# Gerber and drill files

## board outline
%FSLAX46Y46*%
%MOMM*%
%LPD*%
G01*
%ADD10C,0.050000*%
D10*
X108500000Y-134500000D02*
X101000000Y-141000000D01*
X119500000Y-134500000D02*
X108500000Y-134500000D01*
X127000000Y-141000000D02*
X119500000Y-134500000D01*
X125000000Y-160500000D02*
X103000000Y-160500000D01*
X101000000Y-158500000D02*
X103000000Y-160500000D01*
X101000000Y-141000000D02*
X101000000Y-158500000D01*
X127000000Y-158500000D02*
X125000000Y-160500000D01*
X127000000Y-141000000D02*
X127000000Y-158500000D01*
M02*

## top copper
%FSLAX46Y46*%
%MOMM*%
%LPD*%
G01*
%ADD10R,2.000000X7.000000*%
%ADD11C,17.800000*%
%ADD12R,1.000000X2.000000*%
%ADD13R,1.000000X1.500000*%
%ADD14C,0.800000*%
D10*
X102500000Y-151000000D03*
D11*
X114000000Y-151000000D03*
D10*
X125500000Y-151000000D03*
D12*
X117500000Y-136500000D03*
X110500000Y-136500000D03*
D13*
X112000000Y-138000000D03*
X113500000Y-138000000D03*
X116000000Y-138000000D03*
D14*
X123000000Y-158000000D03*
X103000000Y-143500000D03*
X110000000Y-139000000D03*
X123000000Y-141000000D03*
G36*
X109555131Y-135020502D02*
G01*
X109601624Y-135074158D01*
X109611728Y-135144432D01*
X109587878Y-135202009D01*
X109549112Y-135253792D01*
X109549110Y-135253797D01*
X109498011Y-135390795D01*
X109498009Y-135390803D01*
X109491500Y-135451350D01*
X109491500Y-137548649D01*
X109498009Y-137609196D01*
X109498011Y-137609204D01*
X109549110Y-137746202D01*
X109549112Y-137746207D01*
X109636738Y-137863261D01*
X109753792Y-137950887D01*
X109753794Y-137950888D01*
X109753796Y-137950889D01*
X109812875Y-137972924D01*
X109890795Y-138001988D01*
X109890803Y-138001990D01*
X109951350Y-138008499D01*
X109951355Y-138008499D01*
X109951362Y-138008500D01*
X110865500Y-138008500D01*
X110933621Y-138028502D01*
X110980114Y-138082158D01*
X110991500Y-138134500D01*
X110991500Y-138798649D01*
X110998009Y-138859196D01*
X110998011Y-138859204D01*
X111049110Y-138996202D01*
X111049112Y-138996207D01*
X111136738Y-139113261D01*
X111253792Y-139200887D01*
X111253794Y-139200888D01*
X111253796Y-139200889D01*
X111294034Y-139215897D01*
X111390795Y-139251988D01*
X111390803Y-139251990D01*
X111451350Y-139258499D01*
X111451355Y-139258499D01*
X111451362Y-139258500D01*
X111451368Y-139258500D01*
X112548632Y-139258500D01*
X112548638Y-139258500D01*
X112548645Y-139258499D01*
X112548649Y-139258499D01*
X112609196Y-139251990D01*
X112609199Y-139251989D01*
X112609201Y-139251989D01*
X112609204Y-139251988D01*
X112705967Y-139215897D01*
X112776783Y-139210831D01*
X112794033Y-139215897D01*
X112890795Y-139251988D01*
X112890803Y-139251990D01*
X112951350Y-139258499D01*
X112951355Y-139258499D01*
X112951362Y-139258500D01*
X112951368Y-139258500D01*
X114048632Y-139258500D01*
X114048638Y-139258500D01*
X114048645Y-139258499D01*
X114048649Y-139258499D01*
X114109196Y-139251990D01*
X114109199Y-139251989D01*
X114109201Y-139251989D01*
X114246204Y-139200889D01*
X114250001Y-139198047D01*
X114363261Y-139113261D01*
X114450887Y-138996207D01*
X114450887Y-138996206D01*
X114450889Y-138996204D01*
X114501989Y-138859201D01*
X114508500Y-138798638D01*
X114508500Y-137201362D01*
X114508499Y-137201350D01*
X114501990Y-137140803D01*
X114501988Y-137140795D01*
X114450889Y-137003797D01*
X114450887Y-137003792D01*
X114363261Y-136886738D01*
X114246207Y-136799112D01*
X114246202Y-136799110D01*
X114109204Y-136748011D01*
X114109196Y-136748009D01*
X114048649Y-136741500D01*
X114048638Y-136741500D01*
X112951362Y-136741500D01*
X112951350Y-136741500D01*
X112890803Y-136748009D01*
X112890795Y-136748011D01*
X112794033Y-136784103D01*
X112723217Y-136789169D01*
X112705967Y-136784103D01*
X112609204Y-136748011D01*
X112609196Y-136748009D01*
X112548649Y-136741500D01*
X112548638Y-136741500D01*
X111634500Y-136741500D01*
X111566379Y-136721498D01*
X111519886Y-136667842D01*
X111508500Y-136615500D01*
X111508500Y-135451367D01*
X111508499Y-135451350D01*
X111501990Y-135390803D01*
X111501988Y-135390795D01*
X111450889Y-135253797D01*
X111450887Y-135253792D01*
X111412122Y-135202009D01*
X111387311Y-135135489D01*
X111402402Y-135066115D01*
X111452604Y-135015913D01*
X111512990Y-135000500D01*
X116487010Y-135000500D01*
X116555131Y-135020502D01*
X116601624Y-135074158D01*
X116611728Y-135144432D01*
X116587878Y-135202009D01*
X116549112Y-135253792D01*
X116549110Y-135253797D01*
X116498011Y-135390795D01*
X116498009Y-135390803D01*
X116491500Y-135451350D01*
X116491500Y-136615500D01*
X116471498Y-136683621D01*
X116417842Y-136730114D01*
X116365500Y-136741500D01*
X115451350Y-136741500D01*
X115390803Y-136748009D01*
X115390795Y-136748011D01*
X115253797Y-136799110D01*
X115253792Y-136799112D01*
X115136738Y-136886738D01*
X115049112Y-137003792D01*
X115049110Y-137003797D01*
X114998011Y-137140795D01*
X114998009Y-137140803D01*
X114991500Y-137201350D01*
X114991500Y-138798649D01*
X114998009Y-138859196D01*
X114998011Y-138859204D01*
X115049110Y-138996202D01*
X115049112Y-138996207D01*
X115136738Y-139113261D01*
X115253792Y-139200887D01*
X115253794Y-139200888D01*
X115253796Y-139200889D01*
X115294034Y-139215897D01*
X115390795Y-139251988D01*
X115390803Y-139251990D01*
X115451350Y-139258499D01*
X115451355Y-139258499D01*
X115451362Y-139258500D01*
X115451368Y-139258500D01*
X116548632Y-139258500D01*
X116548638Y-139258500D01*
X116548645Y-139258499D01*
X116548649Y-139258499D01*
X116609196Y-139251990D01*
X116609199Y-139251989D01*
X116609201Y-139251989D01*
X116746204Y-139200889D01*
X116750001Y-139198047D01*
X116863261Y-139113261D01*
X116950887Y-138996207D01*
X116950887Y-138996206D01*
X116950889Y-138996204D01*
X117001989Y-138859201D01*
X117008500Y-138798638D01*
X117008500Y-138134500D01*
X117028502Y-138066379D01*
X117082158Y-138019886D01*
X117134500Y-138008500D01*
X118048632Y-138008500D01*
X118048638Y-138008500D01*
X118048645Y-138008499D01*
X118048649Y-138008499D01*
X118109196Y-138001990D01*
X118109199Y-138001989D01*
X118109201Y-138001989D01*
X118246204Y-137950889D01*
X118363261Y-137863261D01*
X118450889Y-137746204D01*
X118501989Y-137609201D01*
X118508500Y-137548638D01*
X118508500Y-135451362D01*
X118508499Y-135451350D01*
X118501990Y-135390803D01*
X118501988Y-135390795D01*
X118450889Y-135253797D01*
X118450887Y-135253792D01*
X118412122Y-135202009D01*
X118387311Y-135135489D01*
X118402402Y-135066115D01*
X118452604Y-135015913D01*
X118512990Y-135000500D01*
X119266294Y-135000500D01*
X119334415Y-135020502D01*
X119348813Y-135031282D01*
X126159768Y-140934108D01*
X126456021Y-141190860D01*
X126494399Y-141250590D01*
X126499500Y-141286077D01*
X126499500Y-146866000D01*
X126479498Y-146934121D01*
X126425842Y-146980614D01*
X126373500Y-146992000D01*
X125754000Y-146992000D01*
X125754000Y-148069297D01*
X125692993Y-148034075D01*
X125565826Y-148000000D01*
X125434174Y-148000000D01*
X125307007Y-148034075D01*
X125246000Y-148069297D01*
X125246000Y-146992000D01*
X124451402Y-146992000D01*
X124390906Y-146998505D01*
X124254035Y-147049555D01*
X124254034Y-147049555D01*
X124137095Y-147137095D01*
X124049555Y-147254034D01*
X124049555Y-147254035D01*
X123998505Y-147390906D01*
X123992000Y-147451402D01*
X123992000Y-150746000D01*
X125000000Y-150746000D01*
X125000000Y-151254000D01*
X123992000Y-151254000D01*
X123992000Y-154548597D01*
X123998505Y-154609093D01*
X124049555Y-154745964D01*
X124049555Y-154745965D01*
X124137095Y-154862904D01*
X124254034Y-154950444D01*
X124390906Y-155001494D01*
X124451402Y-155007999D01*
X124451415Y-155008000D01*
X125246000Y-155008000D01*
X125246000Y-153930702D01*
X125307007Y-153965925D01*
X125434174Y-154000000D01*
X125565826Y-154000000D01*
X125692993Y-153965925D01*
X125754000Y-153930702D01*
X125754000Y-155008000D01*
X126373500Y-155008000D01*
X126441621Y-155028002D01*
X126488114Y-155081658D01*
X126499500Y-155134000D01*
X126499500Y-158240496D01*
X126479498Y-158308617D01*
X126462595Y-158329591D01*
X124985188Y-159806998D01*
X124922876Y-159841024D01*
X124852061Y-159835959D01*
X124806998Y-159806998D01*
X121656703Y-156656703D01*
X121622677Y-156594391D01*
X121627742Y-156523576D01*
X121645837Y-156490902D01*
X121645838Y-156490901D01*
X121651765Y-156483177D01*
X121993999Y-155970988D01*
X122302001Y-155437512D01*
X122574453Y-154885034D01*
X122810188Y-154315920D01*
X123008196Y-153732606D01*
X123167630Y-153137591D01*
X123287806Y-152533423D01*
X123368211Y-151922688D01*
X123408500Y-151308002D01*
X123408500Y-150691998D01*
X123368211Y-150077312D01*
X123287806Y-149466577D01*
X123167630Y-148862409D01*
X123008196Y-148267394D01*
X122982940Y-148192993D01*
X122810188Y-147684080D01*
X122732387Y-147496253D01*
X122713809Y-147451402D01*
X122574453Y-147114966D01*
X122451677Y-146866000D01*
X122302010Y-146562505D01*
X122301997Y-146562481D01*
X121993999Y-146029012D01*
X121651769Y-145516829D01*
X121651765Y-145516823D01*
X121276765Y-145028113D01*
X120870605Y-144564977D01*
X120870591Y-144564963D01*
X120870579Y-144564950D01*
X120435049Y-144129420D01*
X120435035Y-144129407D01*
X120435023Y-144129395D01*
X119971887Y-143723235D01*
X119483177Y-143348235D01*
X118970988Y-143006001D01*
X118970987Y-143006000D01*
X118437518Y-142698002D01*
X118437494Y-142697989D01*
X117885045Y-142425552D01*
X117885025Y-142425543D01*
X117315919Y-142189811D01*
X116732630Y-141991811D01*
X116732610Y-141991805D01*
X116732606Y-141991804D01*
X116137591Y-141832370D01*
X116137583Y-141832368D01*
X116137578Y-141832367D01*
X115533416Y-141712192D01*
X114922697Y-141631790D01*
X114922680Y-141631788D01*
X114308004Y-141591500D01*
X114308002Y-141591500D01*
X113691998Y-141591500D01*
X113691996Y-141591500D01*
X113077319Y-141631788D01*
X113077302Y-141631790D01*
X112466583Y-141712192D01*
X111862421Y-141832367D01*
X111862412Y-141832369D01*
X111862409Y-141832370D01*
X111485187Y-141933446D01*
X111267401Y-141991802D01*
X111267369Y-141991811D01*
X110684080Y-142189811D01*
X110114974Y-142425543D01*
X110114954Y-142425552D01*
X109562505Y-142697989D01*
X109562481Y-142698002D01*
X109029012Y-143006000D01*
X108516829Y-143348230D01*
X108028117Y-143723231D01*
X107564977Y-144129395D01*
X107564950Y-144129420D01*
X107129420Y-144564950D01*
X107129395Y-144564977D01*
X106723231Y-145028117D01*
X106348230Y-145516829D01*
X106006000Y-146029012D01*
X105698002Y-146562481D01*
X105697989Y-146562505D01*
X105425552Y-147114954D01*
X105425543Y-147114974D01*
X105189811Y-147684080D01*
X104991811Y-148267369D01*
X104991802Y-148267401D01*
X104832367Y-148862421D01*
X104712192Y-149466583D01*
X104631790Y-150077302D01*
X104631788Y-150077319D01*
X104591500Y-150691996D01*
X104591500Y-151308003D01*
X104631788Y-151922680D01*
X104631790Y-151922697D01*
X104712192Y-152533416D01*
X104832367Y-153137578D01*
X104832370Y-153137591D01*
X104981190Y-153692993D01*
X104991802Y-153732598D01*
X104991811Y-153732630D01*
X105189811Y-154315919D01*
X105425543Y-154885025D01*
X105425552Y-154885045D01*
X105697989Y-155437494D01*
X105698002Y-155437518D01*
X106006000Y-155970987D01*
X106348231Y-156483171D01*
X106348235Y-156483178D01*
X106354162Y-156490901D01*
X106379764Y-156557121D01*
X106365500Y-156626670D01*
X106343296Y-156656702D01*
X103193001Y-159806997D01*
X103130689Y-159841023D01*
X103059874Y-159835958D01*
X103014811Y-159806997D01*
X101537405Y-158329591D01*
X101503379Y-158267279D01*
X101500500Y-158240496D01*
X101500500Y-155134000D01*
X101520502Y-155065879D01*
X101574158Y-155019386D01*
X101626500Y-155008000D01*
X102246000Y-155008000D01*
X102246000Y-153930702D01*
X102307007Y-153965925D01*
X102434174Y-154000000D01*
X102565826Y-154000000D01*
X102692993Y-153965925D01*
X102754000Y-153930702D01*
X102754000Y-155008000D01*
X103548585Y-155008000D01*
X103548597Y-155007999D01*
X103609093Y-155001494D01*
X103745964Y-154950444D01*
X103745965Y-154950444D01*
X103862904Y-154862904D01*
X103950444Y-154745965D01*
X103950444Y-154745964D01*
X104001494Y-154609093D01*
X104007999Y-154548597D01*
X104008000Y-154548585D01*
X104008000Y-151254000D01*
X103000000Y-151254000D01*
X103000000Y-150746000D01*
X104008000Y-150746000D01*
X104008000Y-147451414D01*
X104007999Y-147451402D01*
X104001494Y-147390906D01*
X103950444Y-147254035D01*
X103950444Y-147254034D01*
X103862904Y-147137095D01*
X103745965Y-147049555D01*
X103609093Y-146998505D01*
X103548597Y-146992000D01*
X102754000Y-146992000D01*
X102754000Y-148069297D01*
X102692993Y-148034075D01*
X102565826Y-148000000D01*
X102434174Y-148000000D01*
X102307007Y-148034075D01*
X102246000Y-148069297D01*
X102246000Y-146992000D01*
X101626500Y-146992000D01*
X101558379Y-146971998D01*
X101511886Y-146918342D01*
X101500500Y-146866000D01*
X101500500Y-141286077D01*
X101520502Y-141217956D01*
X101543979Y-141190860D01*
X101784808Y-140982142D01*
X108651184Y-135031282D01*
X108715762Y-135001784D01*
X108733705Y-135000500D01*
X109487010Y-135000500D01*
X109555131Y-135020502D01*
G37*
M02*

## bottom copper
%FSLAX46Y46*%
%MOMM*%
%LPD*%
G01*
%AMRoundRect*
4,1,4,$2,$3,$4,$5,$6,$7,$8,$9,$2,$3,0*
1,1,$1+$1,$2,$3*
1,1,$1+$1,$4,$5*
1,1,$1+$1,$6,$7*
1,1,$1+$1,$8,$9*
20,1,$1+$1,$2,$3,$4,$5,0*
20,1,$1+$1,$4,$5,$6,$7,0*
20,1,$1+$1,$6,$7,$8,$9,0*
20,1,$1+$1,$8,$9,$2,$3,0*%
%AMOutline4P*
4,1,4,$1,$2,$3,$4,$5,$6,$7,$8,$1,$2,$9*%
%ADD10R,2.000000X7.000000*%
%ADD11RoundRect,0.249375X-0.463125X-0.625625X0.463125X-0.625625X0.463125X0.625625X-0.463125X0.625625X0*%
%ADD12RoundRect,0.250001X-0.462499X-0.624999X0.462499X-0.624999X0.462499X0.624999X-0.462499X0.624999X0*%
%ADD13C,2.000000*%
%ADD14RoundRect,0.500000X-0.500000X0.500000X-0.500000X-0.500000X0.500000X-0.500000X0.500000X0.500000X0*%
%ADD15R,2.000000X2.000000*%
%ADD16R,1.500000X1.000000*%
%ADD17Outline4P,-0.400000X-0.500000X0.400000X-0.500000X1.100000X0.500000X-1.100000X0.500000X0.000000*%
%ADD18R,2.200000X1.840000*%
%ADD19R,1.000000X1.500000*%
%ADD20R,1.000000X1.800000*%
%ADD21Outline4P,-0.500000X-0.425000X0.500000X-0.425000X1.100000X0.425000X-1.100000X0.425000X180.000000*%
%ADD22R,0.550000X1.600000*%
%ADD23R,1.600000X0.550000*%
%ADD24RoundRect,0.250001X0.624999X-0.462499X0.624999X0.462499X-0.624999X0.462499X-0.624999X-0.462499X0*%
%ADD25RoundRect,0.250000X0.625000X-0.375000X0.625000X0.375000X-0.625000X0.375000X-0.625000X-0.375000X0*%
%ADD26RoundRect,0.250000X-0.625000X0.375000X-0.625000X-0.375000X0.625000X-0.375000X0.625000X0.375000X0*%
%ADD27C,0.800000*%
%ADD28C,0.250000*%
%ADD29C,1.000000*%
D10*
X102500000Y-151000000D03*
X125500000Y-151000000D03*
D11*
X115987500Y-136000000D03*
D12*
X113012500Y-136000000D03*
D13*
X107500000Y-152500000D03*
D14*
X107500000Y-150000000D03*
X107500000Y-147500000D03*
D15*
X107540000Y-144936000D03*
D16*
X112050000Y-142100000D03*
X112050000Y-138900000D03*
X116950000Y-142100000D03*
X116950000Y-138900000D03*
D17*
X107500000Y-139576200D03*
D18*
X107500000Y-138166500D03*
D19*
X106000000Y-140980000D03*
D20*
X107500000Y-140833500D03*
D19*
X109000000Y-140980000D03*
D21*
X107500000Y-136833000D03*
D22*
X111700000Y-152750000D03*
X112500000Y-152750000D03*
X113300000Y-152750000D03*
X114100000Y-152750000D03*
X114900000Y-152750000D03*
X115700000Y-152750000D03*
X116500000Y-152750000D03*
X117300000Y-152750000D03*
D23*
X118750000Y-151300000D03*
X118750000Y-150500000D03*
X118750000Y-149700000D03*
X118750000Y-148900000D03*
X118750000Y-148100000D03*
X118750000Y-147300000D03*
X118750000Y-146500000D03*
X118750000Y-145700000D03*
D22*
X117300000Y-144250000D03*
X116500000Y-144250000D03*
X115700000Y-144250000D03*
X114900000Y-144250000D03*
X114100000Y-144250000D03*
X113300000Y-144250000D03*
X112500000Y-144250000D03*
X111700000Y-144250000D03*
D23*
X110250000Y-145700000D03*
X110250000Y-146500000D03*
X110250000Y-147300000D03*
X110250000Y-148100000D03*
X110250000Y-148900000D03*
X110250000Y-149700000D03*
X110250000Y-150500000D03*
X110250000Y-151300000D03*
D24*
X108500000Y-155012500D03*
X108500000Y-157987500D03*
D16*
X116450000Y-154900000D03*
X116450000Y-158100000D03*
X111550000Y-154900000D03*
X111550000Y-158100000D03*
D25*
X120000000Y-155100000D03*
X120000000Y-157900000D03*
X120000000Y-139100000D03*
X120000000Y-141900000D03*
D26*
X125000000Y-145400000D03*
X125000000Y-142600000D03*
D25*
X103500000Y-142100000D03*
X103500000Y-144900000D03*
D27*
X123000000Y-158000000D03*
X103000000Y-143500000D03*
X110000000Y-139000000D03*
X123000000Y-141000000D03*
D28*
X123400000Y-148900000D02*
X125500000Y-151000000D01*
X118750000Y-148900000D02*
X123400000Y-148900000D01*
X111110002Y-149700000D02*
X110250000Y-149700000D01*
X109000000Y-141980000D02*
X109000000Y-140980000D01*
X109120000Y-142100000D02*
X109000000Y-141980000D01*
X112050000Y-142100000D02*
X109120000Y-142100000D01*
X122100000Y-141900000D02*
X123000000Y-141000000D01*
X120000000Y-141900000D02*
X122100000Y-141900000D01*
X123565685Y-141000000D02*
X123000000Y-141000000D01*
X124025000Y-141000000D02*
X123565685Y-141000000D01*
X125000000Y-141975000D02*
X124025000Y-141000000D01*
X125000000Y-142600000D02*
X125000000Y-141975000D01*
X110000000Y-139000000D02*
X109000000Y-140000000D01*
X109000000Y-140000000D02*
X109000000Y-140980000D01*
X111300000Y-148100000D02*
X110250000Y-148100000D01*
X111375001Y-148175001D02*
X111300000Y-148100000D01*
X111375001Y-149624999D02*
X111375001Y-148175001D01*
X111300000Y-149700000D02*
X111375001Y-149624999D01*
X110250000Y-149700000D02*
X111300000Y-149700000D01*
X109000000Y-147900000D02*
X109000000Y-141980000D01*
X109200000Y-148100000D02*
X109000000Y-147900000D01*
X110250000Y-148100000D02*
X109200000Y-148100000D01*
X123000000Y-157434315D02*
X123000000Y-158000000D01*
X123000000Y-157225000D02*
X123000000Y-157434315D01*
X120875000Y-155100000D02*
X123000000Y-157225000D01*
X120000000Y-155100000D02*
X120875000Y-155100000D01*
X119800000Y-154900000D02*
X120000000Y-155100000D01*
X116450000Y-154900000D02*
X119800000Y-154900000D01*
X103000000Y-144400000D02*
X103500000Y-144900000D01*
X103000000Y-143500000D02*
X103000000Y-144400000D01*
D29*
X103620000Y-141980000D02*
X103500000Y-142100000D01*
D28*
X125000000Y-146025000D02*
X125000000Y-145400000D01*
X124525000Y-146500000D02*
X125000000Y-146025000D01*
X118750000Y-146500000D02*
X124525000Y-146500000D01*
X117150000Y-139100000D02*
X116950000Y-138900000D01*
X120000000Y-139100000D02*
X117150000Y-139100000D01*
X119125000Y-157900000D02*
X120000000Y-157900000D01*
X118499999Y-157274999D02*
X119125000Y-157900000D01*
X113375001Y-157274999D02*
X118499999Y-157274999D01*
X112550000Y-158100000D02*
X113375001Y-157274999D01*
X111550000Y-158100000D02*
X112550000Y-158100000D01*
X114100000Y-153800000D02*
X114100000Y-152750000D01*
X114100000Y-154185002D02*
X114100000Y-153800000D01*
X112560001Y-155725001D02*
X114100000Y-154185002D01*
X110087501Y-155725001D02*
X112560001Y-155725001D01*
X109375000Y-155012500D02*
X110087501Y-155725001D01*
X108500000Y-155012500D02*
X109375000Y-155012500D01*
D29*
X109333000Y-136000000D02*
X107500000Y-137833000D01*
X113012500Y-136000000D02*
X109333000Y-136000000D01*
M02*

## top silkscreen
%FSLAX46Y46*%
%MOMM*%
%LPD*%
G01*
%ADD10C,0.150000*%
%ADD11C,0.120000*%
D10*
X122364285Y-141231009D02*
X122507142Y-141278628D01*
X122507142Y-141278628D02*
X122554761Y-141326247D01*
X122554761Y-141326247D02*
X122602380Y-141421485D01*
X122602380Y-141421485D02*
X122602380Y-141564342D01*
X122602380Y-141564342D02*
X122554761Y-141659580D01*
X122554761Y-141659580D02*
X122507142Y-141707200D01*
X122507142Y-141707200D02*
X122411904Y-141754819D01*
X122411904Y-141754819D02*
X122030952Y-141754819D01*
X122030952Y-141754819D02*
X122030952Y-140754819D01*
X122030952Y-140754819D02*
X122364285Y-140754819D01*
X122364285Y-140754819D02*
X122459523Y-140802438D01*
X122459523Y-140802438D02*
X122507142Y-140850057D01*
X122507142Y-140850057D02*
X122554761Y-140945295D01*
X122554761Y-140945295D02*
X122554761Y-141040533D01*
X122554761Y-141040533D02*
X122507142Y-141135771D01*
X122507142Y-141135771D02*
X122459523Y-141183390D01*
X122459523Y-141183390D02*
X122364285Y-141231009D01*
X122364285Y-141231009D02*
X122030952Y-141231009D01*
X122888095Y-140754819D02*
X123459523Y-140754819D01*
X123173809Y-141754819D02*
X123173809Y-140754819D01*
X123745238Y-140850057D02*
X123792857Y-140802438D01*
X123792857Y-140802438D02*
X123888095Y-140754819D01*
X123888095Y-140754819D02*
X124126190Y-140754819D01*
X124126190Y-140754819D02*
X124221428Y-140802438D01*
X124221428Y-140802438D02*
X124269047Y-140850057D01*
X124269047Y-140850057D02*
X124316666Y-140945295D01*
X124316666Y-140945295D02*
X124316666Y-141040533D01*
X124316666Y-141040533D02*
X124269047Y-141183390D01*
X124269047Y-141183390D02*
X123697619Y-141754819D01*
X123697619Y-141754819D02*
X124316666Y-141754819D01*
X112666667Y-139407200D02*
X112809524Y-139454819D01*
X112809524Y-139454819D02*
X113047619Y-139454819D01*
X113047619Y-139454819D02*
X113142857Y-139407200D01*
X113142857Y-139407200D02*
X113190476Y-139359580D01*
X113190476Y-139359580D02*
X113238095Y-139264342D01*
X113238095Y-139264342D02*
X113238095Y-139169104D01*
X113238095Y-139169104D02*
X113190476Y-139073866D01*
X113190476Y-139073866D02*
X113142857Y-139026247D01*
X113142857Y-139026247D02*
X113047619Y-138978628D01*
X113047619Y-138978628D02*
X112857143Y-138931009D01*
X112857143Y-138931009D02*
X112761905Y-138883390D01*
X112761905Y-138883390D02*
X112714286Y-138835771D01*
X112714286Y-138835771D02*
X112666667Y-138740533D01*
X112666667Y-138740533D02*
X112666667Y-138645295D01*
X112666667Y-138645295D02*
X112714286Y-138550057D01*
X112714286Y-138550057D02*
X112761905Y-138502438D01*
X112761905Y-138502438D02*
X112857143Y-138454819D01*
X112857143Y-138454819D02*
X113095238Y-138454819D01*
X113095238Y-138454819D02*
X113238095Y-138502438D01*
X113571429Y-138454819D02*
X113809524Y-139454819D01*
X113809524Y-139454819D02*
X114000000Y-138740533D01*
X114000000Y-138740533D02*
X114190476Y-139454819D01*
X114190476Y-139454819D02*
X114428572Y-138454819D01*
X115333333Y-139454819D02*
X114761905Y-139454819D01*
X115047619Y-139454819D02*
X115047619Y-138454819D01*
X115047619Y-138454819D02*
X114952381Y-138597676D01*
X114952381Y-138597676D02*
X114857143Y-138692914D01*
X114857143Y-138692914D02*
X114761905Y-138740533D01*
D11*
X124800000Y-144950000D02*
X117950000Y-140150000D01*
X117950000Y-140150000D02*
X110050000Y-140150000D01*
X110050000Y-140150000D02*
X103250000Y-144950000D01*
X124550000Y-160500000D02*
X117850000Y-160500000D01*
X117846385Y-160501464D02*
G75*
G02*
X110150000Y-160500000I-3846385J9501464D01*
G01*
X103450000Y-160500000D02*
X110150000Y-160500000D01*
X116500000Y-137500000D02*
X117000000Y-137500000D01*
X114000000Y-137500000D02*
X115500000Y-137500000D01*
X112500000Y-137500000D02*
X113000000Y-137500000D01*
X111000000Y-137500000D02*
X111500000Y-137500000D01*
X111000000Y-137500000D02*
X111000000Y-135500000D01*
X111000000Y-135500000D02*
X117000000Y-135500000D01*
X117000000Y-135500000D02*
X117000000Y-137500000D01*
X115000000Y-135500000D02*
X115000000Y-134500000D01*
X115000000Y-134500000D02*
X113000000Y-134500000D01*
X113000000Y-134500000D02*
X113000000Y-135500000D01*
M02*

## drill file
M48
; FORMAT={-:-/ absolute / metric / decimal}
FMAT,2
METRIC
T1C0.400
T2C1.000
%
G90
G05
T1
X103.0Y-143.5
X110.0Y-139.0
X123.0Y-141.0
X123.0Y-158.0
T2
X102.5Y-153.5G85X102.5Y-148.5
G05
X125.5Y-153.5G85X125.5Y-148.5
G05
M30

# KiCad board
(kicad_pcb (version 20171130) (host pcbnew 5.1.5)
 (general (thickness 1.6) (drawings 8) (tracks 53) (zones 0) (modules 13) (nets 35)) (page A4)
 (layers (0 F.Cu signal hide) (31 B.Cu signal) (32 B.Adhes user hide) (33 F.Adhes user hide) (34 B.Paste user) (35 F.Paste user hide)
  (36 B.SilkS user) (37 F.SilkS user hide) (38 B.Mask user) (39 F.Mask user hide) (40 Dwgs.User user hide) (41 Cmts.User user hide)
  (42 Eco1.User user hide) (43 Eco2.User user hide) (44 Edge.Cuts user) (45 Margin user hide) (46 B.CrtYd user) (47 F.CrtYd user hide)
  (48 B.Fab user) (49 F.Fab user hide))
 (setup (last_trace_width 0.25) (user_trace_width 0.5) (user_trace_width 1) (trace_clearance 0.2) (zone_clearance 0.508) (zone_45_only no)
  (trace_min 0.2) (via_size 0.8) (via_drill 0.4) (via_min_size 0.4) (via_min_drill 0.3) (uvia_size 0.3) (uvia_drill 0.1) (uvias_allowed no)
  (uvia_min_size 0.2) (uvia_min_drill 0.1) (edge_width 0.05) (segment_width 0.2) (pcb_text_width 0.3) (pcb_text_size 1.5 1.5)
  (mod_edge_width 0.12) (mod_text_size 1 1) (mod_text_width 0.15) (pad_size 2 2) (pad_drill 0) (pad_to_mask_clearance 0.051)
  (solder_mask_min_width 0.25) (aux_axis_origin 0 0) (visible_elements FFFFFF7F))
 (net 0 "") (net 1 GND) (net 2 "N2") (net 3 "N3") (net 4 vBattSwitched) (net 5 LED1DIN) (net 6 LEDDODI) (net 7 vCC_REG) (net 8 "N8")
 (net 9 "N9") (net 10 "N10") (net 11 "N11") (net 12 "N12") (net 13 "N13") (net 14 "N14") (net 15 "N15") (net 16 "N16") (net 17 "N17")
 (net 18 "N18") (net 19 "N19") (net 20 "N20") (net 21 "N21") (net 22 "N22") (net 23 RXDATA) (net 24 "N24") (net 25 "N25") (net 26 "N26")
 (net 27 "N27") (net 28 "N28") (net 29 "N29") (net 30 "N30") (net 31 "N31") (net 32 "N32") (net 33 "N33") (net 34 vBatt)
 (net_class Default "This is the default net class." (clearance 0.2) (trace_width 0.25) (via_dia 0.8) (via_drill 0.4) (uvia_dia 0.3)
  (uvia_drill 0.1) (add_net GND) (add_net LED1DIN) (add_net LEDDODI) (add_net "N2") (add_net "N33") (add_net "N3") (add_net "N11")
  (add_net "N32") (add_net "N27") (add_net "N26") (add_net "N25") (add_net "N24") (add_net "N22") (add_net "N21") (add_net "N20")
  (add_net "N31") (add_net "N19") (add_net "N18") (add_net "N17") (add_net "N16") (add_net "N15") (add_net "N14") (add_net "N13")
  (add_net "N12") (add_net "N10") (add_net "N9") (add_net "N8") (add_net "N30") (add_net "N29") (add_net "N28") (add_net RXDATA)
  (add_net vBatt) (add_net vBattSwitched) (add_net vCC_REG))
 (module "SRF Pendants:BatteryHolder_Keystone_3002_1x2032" (layer F.Cu) (at 114 151 180)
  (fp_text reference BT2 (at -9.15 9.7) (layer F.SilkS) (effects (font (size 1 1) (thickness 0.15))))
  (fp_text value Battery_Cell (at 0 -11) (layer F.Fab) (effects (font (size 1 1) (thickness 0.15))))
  (fp_line (start -10.8 6.05) (end -3.95 10.85) (layer F.SilkS) (width 0.12))
  (fp_line (start -3.95 10.85) (end 3.95 10.85) (layer F.SilkS) (width 0.12))
  (fp_line (start 3.95 10.85) (end 10.75 6.05) (layer F.SilkS) (width 0.12))
  (fp_line (start -10.55 -9.5) (end -3.85 -9.5) (layer F.SilkS) (width 0.12))
  (fp_arc (start 0 0) (end 3.85 -9.5) (angle -44.1) (layer F.SilkS) (width 0.12))
  (fp_line (start 10.55 -9.5) (end 3.85 -9.5) (layer F.SilkS) (width 0.12))
  (pad 1 thru_hole rect (at 11.5 0 180) (size 2 7) (drill oval 1 6) (layers *.Cu *.Mask) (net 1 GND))
  (pad 2 smd circle (at 0 0 180) (size 17.8 17.8) (layers F.Cu F.Mask) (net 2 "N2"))
  (pad 1 thru_hole rect (at -11.5 0 180) (size 2 7) (drill oval 1 6) (layers *.Cu *.Mask) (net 1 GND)))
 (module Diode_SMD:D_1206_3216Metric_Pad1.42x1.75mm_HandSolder (layer B.Cu) (at 114.5 136)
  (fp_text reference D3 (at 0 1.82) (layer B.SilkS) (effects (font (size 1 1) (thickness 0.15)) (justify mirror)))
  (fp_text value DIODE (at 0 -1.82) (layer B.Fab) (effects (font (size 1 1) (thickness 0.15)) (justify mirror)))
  (pad 2 smd roundrect (at 1.4875 0) (size 1.425 1.75) (layers B.Cu B.Paste B.Mask) (roundrect_rratio 0.175) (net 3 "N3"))
  (pad 1 smd roundrect (at -1.4875 0) (size 1.425 1.75) (layers B.Cu B.Paste B.Mask) (roundrect_rratio 0.175439) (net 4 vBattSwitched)))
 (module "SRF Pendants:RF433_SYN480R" (layer B.Cu) (at 105 149 270)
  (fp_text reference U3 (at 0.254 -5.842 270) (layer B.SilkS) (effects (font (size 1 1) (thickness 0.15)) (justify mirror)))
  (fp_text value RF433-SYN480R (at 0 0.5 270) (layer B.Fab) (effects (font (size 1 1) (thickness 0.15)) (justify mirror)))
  (pad 4 smd circle (at 3.5 -2.5 270) (size 2 2) (layers B.Cu B.Paste B.Mask) (thermal_gap 0.5))
  (pad 3 smd roundrect (at 1 -2.5 270) (size 2 2) (layers B.Cu B.Paste B.Mask) (roundrect_rratio 0.25))
  (pad 2 smd roundrect (at -1.5 -2.5 270) (size 2 2) (layers B.Cu B.Paste B.Mask) (roundrect_rratio 0.25))
  (pad 1 smd rect (at -4.064 -2.54 270) (size 2 2) (layers B.Cu B.Paste B.Mask)))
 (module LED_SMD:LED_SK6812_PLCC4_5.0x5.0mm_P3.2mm (layer B.Cu) (at 114.5 140.5)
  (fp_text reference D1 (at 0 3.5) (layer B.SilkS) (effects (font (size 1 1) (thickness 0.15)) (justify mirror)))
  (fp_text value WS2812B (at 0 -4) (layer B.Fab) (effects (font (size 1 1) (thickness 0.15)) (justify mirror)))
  (pad 3 smd rect (at -2.45 1.6) (size 1.5 1) (layers B.Cu B.Paste B.Mask) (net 1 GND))
  (pad 4 smd rect (at -2.45 -1.6) (size 1.5 1) (layers B.Cu B.Paste B.Mask) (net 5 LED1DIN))
  (pad 2 smd rect (at 2.45 1.6) (size 1.5 1) (layers B.Cu B.Paste B.Mask) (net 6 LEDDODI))
  (pad 1 smd rect (at 2.45 -1.6) (size 1.5 1) (layers B.Cu B.Paste B.Mask) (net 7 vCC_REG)))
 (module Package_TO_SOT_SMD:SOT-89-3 (layer B.Cu) (at 107.5 139.5 90)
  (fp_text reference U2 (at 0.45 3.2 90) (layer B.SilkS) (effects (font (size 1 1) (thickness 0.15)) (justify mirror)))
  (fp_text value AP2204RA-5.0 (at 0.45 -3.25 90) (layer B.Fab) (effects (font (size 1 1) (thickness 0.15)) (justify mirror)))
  (pad 2 smd trapezoid (at -0.0762 0) (size 1.5 1) (rect_delta 0 -0.7) (layers B.Cu B.Paste B.Mask) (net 3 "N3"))
  (pad 2 smd rect (at 1.3335 0 180) (size 2.2 1.84) (layers B.Cu B.Paste B.Mask) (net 3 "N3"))
  (pad 3 smd rect (at -1.48 -1.5 180) (size 1 1.5) (layers B.Cu B.Paste B.Mask) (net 7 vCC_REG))
  (pad 2 smd rect (at -1.3335 0 180) (size 1 1.8) (layers B.Cu B.Paste B.Mask) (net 3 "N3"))
  (pad 1 smd rect (at -1.48 1.5 180) (size 1 1.5) (layers B.Cu B.Paste B.Mask) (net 1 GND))
  (pad 2 smd trapezoid (at 2.667 0 180) (size 1.6 0.85) (rect_delta 0 -0.6) (layers B.Cu B.Paste B.Mask) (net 3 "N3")))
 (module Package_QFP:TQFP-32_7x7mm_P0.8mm (layer B.Cu) (at 114.5 148.5)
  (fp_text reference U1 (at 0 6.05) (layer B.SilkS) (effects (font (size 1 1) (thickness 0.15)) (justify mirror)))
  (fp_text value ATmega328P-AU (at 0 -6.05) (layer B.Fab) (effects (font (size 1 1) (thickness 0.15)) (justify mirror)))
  (pad 32 smd rect (at -2.8 4.25 270) (size 1.6 0.55) (layers B.Cu B.Paste B.Mask) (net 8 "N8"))
  (pad 31 smd rect (at -2 4.25 270) (size 1.6 0.55) (layers B.Cu B.Paste B.Mask) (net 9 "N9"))
  (pad 30 smd rect (at -1.2 4.25 270) (size 1.6 0.55) (layers B.Cu B.Paste B.Mask) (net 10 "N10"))
  (pad 29 smd rect (at -0.4 4.25 270) (size 1.6 0.55) (layers B.Cu B.Paste B.Mask) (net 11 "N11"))
  (pad 28 smd rect (at 0.4 4.25 270) (size 1.6 0.55) (layers B.Cu B.Paste B.Mask) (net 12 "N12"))
  (pad 27 smd rect (at 1.2 4.25 270) (size 1.6 0.55) (layers B.Cu B.Paste B.Mask) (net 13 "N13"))
  (pad 26 smd rect (at 2 4.25 270) (size 1.6 0.55) (layers B.Cu B.Paste B.Mask) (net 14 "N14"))
  (pad 25 smd rect (at 2.8 4.25 270) (size 1.6 0.55) (layers B.Cu B.Paste B.Mask) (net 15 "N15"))
  (pad 24 smd rect (at 4.25 2.8) (size 1.6 0.55) (layers B.Cu B.Paste B.Mask) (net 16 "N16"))
  (pad 23 smd rect (at 4.25 2) (size 1.6 0.55) (layers B.Cu B.Paste B.Mask) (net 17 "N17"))
  (pad 22 smd rect (at 4.25 1.2) (size 1.6 0.55) (layers B.Cu B.Paste B.Mask) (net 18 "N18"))
  (pad 21 smd rect (at 4.25 0.4) (size 1.6 0.55) (layers B.Cu B.Paste B.Mask) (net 1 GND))
  (pad 20 smd rect (at 4.25 -0.4) (size 1.6 0.55) (layers B.Cu B.Paste B.Mask) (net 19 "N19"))
  (pad 19 smd rect (at 4.25 -1.2) (size 1.6 0.55) (layers B.Cu B.Paste B.Mask) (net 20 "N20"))
  (pad 18 smd rect (at 4.25 -2) (size 1.6 0.55) (layers B.Cu B.Paste B.Mask) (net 7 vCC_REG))
  (pad 17 smd rect (at 4.25 -2.8) (size 1.6 0.55) (layers B.Cu B.Paste B.Mask) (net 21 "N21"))
  (pad 16 smd rect (at 2.8 -4.25 270) (size 1.6 0.55) (layers B.Cu B.Paste B.Mask) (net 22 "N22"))
  (pad 15 smd rect (at 2 -4.25 270) (size 1.6 0.55) (layers B.Cu B.Paste B.Mask) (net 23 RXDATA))
  (pad 14 smd rect (at 1.2 -4.25 270) (size 1.6 0.55) (layers B.Cu B.Paste B.Mask) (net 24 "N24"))
  (pad 13 smd rect (at 0.4 -4.25 270) (size 1.6 0.55) (layers B.Cu B.Paste B.Mask) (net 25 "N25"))
  (pad 12 smd rect (at -0.4 -4.25 270) (size 1.6 0.55) (layers B.Cu B.Paste B.Mask) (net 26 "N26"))
  (pad 11 smd rect (at -1.2 -4.25 270) (size 1.6 0.55) (layers B.Cu B.Paste B.Mask) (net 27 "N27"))
  (pad 10 smd rect (at -2 -4.25 270) (size 1.6 0.55) (layers B.Cu B.Paste B.Mask) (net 5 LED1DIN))
  (pad 9 smd rect (at -2.8 -4.25 270) (size 1.6 0.55) (layers B.Cu B.Paste B.Mask) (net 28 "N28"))
  (pad 8 smd rect (at -4.25 -2.8) (size 1.6 0.55) (layers B.Cu B.Paste B.Mask) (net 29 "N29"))
  (pad 7 smd rect (at -4.25 -2) (size 1.6 0.55) (layers B.Cu B.Paste B.Mask) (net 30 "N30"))
  (pad 6 smd rect (at -4.25 -1.2) (size 1.6 0.55) (layers B.Cu B.Paste B.Mask) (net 7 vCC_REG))
  (pad 5 smd rect (at -4.25 -0.4) (size 1.6 0.55) (layers B.Cu B.Paste B.Mask) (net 1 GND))
  (pad 4 smd rect (at -4.25 0.4) (size 1.6 0.55) (layers B.Cu B.Paste B.Mask) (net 7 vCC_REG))
  (pad 3 smd rect (at -4.25 1.2) (size 1.6 0.55) (layers B.Cu B.Paste B.Mask) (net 1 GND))
  (pad 2 smd rect (at -4.25 2) (size 1.6 0.55) (layers B.Cu B.Paste B.Mask) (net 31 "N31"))
  (pad 1 smd rect (at -4.25 2.8) (size 1.6 0.55) (layers B.Cu B.Paste B.Mask) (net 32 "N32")))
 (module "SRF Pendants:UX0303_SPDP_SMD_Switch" (layer F.Cu) (at 114 139.5 180)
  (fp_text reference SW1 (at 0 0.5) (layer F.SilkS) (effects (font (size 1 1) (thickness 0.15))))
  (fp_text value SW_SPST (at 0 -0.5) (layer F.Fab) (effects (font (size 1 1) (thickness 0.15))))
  (fp_line (start -2.5 2) (end -3 2) (layer F.SilkS) (width 0.12))
  (fp_line (start 0 2) (end -1.5 2) (layer F.SilkS) (width 0.12))
  (fp_line (start 1.5 2) (end 1 2) (layer F.SilkS) (width 0.12))
  (fp_line (start 3 2) (end 2.5 2) (layer F.SilkS) (width 0.12)) (fp_line (start 3 2) (end 3 4) (layer F.SilkS) (width 0.12))
  (fp_line (start 3 4) (end -3 4) (layer F.SilkS) (width 0.12))
  (fp_line (start -3 4) (end -3 2) (layer F.SilkS) (width 0.12))
  (fp_line (start -1 4) (end -1 5) (layer F.SilkS) (width 0.12))
  (fp_line (start -1 5) (end 1 5) (layer F.SilkS) (width 0.12)) (fp_line (start 1 5) (end 1 4) (layer F.SilkS) (width 0.12))
  (pad X smd rect (at -3.5 3 180) (size 1 2) (layers F.Cu F.Paste F.Mask))
  (pad X smd rect (at 3.5 3 180) (size 1 2) (layers F.Cu F.Paste F.Mask))
  (pad 1 smd rect (at 2 1.5 180) (size 1 1.5) (layers F.Cu F.Paste F.Mask) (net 2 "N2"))
  (pad 2 smd rect (at 0.5 1.5 180) (size 1 1.5) (layers F.Cu F.Paste F.Mask) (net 4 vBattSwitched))
  (pad 3 smd rect (at -2 1.5 180) (size 1 1.5) (layers F.Cu F.Paste F.Mask)))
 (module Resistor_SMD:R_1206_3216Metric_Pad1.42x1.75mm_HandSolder (layer B.Cu) (at 108.5 156.5 90)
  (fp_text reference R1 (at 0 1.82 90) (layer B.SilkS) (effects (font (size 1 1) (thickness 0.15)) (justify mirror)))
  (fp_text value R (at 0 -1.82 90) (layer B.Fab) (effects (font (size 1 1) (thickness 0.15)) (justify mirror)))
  (pad 2 smd roundrect (at 1.4875 0 90) (size 1.425 1.75) (layers B.Cu B.Paste B.Mask) (roundrect_rratio 0.175439) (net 11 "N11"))
  (pad 1 smd roundrect (at -1.4875 0 90) (size 1.425 1.75) (layers B.Cu B.Paste B.Mask) (roundrect_rratio 0.175439) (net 7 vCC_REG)))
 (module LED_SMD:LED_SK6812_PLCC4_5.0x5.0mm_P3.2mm (layer B.Cu) (at 114 156.5 180)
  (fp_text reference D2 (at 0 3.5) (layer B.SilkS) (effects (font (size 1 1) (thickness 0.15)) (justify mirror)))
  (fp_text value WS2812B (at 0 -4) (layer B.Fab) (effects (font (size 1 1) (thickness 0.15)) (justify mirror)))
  (pad 3 smd rect (at -2.45 1.6 180) (size 1.5 1) (layers B.Cu B.Paste B.Mask) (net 1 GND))
  (pad 4 smd rect (at -2.45 -1.6 180) (size 1.5 1) (layers B.Cu B.Paste B.Mask) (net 6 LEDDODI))
  (pad 2 smd rect (at 2.45 1.6 180) (size 1.5 1) (layers B.Cu B.Paste B.Mask) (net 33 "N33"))
  (pad 1 smd rect (at 2.45 -1.6 180) (size 1.5 1) (layers B.Cu B.Paste B.Mask) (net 7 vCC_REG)))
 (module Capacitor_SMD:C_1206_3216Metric (layer B.Cu) (at 120 156.5 90)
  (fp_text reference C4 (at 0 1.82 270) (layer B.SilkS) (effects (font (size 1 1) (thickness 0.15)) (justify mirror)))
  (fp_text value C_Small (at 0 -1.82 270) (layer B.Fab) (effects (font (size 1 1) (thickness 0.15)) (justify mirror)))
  (pad 2 smd roundrect (at 1.4 0 90) (size 1.25 1.75) (layers B.Cu B.Paste B.Mask) (roundrect_rratio 0.2) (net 1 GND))
  (pad 1 smd roundrect (at -1.4 0 90) (size 1.25 1.75) (layers B.Cu B.Paste B.Mask) (roundrect_rratio 0.2) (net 7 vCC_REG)))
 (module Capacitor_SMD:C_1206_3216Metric (layer B.Cu) (at 120 140.5 90)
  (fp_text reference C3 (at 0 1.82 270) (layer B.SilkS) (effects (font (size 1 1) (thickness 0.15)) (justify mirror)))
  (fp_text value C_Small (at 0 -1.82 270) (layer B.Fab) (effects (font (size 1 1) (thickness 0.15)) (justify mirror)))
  (pad 2 smd roundrect (at 1.4 0 90) (size 1.25 1.75) (layers B.Cu B.Paste B.Mask) (roundrect_rratio 0.2) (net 7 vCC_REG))
  (pad 1 smd roundrect (at -1.4 0 90) (size 1.25 1.75) (layers B.Cu B.Paste B.Mask) (roundrect_rratio 0.2) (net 1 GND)))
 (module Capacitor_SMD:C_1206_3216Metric (layer B.Cu) (at 125 144 270)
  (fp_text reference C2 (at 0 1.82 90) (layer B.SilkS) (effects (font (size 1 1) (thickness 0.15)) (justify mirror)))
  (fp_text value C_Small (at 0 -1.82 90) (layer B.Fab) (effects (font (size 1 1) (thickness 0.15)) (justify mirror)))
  (pad 2 smd roundrect (at 1.4 0 270) (size 1.25 1.75) (layers B.Cu B.Paste B.Mask) (roundrect_rratio 0.2) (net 7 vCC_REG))
  (pad 1 smd roundrect (at -1.4 0 270) (size 1.25 1.75) (layers B.Cu B.Paste B.Mask) (roundrect_rratio 0.2) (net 1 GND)))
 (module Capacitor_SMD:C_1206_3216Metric (layer B.Cu) (at 103.5 143.5 90)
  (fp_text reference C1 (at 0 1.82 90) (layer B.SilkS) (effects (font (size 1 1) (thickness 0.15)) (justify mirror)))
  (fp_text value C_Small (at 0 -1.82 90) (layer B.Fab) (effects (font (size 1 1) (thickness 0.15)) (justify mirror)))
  (pad 2 smd roundrect (at 1.4 0 90) (size 1.25 1.75) (layers B.Cu B.Paste B.Mask) (roundrect_rratio 0.2) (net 7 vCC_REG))
  (pad 1 smd roundrect (at -1.4 0 90) (size 1.25 1.75) (layers B.Cu B.Paste B.Mask) (roundrect_rratio 0.2) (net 1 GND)))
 (gr_line (start 108.5 134.5) (end 101 141) (layer Edge.Cuts) (width 0.05))
 (gr_line (start 119.5 134.5) (end 108.5 134.5) (layer Edge.Cuts) (width 0.05))
 (gr_line (start 127 141) (end 119.5 134.5) (layer Edge.Cuts) (width 0.05))
 (gr_line (start 125 160.5) (end 103 160.5) (layer Edge.Cuts) (width 0.05))
 (gr_line (start 101 158.5) (end 103 160.5) (layer Edge.Cuts) (width 0.05))
 (gr_line (start 101 141) (end 101 158.5) (layer Edge.Cuts) (width 0.05))
 (gr_line (start 127 158.5) (end 125 160.5) (layer Edge.Cuts) (width 0.05))
 (gr_line (start 127 141) (end 127 158.5) (layer Edge.Cuts) (width 0.05))
 (via (at 123 158) (size 0.8) (drill 0.4) (layers F.Cu B.Cu) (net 1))
 (via (at 103 143.5) (size 0.8) (drill 0.4) (layers F.Cu B.Cu) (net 1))
 (via (at 110 139) (size 0.8) (drill 0.4) (layers F.Cu B.Cu) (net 1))
 (via (at 123 141) (size 0.8) (drill 0.4) (layers F.Cu B.Cu) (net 1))
 (segment (start 123.4 148.9) (end 125.5 151) (width 0.25) (layer B.Cu) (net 1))
 (segment (start 118.75 148.9) (end 123.4 148.9) (width 0.25) (layer B.Cu) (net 1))
 (segment (start 111.110002 149.7) (end 110.25 149.7) (width 0.25) (layer B.Cu) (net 1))
 (segment (start 109 141.98) (end 109 140.98) (width 0.25) (layer B.Cu) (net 1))
 (segment (start 109.12 142.1) (end 109 141.98) (width 0.25) (layer B.Cu) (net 1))
 (segment (start 112.05 142.1) (end 109.12 142.1) (width 0.25) (layer B.Cu) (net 1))
 (segment (start 122.1 141.9) (end 123 141) (width 0.25) (layer B.Cu) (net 1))
 (segment (start 120 141.9) (end 122.1 141.9) (width 0.25) (layer B.Cu) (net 1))
 (segment (start 123.565685 141) (end 123 141) (width 0.25) (layer B.Cu) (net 1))
 (segment (start 124.025 141) (end 123.565685 141) (width 0.25) (layer B.Cu) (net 1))
 (segment (start 125 141.975) (end 124.025 141) (width 0.25) (layer B.Cu) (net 1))
 (segment (start 125 142.6) (end 125 141.975) (width 0.25) (layer B.Cu) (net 1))
 (segment (start 110 139) (end 109 140) (width 0.25) (layer B.Cu) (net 1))
 (segment (start 109 140) (end 109 140.98) (width 0.25) (layer B.Cu) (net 1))
 (segment (start 111.3 148.1) (end 110.25 148.1) (width 0.25) (layer B.Cu) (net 1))
 (segment (start 111.375001 148.175001) (end 111.3 148.1) (width 0.25) (layer B.Cu) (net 1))
 (segment (start 111.375001 149.624999) (end 111.375001 148.175001) (width 0.25) (layer B.Cu) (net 1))
 (segment (start 111.3 149.7) (end 111.375001 149.624999) (width 0.25) (layer B.Cu) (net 1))
 (segment (start 110.25 149.7) (end 111.3 149.7) (width 0.25) (layer B.Cu) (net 1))
 (segment (start 109 147.9) (end 109 141.98) (width 0.25) (layer B.Cu) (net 1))
 (segment (start 109.2 148.1) (end 109 147.9) (width 0.25) (layer B.Cu) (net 1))
 (segment (start 110.25 148.1) (end 109.2 148.1) (width 0.25) (layer B.Cu) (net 1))
 (segment (start 123 157.434315) (end 123 158) (width 0.25) (layer B.Cu) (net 1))
 (segment (start 123 157.225) (end 123 157.434315) (width 0.25) (layer B.Cu) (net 1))
 (segment (start 120.875 155.1) (end 123 157.225) (width 0.25) (layer B.Cu) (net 1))
 (segment (start 120 155.1) (end 120.875 155.1) (width 0.25) (layer B.Cu) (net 1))
 (segment (start 119.8 154.9) (end 120 155.1) (width 0.25) (layer B.Cu) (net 1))
 (segment (start 116.45 154.9) (end 119.8 154.9) (width 0.25) (layer B.Cu) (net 1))
 (segment (start 103 144.4) (end 103.5 144.9) (width 0.25) (layer B.Cu) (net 1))
 (segment (start 103 143.5) (end 103 144.4) (width 0.25) (layer B.Cu) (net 1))
 (segment (start 103.62 141.98) (end 103.5 142.1) (width 1) (layer B.Cu) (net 7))
 (segment (start 125 146.025) (end 125 145.4) (width 0.25) (layer B.Cu) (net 7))
 (segment (start 124.525 146.5) (end 125 146.025) (width 0.25) (layer B.Cu) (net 7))
 (segment (start 118.75 146.5) (end 124.525 146.5) (width 0.25) (layer B.Cu) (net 7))
 (segment (start 117.15 139.1) (end 116.95 138.9) (width 0.25) (layer B.Cu) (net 7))
 (segment (start 120 139.1) (end 117.15 139.1) (width 0.25) (layer B.Cu) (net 7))
 (segment (start 119.125 157.9) (end 120 157.9) (width 0.25) (layer B.Cu) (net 7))
 (segment (start 118.499999 157.274999) (end 119.125 157.9) (width 0.25) (layer B.Cu) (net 7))
 (segment (start 113.375001 157.274999) (end 118.499999 157.274999) (width 0.25) (layer B.Cu) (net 7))
 (segment (start 112.55 158.1) (end 113.375001 157.274999) (width 0.25) (layer B.Cu) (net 7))
 (segment (start 111.55 158.1) (end 112.55 158.1) (width 0.25) (layer B.Cu) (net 7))
 (segment (start 114.1 153.8) (end 114.1 152.75) (width 0.25) (layer B.Cu) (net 11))
 (segment (start 114.1 154.185002) (end 114.1 153.8) (width 0.25) (layer B.Cu) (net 11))
 (segment (start 112.560001 155.725001) (end 114.1 154.185002) (width 0.25) (layer B.Cu) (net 11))
 (segment (start 110.087501 155.725001) (end 112.560001 155.725001) (width 0.25) (layer B.Cu) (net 11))
 (segment (start 109.375 155.0125) (end 110.087501 155.725001) (width 0.25) (layer B.Cu) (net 11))
 (segment (start 108.5 155.0125) (end 109.375 155.0125) (width 0.25) (layer B.Cu) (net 11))
 (segment (start 109.333 136) (end 107.5 137.833) (width 1) (layer B.Cu) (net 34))
 (segment (start 113.0125 136) (end 109.333 136) (width 1) (layer B.Cu) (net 34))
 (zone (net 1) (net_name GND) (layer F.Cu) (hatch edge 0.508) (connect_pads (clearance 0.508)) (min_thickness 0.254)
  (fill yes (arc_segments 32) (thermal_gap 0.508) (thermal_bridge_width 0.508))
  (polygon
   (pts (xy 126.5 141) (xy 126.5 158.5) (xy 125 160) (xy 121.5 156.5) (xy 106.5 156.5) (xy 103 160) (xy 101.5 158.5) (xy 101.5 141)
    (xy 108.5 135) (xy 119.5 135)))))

